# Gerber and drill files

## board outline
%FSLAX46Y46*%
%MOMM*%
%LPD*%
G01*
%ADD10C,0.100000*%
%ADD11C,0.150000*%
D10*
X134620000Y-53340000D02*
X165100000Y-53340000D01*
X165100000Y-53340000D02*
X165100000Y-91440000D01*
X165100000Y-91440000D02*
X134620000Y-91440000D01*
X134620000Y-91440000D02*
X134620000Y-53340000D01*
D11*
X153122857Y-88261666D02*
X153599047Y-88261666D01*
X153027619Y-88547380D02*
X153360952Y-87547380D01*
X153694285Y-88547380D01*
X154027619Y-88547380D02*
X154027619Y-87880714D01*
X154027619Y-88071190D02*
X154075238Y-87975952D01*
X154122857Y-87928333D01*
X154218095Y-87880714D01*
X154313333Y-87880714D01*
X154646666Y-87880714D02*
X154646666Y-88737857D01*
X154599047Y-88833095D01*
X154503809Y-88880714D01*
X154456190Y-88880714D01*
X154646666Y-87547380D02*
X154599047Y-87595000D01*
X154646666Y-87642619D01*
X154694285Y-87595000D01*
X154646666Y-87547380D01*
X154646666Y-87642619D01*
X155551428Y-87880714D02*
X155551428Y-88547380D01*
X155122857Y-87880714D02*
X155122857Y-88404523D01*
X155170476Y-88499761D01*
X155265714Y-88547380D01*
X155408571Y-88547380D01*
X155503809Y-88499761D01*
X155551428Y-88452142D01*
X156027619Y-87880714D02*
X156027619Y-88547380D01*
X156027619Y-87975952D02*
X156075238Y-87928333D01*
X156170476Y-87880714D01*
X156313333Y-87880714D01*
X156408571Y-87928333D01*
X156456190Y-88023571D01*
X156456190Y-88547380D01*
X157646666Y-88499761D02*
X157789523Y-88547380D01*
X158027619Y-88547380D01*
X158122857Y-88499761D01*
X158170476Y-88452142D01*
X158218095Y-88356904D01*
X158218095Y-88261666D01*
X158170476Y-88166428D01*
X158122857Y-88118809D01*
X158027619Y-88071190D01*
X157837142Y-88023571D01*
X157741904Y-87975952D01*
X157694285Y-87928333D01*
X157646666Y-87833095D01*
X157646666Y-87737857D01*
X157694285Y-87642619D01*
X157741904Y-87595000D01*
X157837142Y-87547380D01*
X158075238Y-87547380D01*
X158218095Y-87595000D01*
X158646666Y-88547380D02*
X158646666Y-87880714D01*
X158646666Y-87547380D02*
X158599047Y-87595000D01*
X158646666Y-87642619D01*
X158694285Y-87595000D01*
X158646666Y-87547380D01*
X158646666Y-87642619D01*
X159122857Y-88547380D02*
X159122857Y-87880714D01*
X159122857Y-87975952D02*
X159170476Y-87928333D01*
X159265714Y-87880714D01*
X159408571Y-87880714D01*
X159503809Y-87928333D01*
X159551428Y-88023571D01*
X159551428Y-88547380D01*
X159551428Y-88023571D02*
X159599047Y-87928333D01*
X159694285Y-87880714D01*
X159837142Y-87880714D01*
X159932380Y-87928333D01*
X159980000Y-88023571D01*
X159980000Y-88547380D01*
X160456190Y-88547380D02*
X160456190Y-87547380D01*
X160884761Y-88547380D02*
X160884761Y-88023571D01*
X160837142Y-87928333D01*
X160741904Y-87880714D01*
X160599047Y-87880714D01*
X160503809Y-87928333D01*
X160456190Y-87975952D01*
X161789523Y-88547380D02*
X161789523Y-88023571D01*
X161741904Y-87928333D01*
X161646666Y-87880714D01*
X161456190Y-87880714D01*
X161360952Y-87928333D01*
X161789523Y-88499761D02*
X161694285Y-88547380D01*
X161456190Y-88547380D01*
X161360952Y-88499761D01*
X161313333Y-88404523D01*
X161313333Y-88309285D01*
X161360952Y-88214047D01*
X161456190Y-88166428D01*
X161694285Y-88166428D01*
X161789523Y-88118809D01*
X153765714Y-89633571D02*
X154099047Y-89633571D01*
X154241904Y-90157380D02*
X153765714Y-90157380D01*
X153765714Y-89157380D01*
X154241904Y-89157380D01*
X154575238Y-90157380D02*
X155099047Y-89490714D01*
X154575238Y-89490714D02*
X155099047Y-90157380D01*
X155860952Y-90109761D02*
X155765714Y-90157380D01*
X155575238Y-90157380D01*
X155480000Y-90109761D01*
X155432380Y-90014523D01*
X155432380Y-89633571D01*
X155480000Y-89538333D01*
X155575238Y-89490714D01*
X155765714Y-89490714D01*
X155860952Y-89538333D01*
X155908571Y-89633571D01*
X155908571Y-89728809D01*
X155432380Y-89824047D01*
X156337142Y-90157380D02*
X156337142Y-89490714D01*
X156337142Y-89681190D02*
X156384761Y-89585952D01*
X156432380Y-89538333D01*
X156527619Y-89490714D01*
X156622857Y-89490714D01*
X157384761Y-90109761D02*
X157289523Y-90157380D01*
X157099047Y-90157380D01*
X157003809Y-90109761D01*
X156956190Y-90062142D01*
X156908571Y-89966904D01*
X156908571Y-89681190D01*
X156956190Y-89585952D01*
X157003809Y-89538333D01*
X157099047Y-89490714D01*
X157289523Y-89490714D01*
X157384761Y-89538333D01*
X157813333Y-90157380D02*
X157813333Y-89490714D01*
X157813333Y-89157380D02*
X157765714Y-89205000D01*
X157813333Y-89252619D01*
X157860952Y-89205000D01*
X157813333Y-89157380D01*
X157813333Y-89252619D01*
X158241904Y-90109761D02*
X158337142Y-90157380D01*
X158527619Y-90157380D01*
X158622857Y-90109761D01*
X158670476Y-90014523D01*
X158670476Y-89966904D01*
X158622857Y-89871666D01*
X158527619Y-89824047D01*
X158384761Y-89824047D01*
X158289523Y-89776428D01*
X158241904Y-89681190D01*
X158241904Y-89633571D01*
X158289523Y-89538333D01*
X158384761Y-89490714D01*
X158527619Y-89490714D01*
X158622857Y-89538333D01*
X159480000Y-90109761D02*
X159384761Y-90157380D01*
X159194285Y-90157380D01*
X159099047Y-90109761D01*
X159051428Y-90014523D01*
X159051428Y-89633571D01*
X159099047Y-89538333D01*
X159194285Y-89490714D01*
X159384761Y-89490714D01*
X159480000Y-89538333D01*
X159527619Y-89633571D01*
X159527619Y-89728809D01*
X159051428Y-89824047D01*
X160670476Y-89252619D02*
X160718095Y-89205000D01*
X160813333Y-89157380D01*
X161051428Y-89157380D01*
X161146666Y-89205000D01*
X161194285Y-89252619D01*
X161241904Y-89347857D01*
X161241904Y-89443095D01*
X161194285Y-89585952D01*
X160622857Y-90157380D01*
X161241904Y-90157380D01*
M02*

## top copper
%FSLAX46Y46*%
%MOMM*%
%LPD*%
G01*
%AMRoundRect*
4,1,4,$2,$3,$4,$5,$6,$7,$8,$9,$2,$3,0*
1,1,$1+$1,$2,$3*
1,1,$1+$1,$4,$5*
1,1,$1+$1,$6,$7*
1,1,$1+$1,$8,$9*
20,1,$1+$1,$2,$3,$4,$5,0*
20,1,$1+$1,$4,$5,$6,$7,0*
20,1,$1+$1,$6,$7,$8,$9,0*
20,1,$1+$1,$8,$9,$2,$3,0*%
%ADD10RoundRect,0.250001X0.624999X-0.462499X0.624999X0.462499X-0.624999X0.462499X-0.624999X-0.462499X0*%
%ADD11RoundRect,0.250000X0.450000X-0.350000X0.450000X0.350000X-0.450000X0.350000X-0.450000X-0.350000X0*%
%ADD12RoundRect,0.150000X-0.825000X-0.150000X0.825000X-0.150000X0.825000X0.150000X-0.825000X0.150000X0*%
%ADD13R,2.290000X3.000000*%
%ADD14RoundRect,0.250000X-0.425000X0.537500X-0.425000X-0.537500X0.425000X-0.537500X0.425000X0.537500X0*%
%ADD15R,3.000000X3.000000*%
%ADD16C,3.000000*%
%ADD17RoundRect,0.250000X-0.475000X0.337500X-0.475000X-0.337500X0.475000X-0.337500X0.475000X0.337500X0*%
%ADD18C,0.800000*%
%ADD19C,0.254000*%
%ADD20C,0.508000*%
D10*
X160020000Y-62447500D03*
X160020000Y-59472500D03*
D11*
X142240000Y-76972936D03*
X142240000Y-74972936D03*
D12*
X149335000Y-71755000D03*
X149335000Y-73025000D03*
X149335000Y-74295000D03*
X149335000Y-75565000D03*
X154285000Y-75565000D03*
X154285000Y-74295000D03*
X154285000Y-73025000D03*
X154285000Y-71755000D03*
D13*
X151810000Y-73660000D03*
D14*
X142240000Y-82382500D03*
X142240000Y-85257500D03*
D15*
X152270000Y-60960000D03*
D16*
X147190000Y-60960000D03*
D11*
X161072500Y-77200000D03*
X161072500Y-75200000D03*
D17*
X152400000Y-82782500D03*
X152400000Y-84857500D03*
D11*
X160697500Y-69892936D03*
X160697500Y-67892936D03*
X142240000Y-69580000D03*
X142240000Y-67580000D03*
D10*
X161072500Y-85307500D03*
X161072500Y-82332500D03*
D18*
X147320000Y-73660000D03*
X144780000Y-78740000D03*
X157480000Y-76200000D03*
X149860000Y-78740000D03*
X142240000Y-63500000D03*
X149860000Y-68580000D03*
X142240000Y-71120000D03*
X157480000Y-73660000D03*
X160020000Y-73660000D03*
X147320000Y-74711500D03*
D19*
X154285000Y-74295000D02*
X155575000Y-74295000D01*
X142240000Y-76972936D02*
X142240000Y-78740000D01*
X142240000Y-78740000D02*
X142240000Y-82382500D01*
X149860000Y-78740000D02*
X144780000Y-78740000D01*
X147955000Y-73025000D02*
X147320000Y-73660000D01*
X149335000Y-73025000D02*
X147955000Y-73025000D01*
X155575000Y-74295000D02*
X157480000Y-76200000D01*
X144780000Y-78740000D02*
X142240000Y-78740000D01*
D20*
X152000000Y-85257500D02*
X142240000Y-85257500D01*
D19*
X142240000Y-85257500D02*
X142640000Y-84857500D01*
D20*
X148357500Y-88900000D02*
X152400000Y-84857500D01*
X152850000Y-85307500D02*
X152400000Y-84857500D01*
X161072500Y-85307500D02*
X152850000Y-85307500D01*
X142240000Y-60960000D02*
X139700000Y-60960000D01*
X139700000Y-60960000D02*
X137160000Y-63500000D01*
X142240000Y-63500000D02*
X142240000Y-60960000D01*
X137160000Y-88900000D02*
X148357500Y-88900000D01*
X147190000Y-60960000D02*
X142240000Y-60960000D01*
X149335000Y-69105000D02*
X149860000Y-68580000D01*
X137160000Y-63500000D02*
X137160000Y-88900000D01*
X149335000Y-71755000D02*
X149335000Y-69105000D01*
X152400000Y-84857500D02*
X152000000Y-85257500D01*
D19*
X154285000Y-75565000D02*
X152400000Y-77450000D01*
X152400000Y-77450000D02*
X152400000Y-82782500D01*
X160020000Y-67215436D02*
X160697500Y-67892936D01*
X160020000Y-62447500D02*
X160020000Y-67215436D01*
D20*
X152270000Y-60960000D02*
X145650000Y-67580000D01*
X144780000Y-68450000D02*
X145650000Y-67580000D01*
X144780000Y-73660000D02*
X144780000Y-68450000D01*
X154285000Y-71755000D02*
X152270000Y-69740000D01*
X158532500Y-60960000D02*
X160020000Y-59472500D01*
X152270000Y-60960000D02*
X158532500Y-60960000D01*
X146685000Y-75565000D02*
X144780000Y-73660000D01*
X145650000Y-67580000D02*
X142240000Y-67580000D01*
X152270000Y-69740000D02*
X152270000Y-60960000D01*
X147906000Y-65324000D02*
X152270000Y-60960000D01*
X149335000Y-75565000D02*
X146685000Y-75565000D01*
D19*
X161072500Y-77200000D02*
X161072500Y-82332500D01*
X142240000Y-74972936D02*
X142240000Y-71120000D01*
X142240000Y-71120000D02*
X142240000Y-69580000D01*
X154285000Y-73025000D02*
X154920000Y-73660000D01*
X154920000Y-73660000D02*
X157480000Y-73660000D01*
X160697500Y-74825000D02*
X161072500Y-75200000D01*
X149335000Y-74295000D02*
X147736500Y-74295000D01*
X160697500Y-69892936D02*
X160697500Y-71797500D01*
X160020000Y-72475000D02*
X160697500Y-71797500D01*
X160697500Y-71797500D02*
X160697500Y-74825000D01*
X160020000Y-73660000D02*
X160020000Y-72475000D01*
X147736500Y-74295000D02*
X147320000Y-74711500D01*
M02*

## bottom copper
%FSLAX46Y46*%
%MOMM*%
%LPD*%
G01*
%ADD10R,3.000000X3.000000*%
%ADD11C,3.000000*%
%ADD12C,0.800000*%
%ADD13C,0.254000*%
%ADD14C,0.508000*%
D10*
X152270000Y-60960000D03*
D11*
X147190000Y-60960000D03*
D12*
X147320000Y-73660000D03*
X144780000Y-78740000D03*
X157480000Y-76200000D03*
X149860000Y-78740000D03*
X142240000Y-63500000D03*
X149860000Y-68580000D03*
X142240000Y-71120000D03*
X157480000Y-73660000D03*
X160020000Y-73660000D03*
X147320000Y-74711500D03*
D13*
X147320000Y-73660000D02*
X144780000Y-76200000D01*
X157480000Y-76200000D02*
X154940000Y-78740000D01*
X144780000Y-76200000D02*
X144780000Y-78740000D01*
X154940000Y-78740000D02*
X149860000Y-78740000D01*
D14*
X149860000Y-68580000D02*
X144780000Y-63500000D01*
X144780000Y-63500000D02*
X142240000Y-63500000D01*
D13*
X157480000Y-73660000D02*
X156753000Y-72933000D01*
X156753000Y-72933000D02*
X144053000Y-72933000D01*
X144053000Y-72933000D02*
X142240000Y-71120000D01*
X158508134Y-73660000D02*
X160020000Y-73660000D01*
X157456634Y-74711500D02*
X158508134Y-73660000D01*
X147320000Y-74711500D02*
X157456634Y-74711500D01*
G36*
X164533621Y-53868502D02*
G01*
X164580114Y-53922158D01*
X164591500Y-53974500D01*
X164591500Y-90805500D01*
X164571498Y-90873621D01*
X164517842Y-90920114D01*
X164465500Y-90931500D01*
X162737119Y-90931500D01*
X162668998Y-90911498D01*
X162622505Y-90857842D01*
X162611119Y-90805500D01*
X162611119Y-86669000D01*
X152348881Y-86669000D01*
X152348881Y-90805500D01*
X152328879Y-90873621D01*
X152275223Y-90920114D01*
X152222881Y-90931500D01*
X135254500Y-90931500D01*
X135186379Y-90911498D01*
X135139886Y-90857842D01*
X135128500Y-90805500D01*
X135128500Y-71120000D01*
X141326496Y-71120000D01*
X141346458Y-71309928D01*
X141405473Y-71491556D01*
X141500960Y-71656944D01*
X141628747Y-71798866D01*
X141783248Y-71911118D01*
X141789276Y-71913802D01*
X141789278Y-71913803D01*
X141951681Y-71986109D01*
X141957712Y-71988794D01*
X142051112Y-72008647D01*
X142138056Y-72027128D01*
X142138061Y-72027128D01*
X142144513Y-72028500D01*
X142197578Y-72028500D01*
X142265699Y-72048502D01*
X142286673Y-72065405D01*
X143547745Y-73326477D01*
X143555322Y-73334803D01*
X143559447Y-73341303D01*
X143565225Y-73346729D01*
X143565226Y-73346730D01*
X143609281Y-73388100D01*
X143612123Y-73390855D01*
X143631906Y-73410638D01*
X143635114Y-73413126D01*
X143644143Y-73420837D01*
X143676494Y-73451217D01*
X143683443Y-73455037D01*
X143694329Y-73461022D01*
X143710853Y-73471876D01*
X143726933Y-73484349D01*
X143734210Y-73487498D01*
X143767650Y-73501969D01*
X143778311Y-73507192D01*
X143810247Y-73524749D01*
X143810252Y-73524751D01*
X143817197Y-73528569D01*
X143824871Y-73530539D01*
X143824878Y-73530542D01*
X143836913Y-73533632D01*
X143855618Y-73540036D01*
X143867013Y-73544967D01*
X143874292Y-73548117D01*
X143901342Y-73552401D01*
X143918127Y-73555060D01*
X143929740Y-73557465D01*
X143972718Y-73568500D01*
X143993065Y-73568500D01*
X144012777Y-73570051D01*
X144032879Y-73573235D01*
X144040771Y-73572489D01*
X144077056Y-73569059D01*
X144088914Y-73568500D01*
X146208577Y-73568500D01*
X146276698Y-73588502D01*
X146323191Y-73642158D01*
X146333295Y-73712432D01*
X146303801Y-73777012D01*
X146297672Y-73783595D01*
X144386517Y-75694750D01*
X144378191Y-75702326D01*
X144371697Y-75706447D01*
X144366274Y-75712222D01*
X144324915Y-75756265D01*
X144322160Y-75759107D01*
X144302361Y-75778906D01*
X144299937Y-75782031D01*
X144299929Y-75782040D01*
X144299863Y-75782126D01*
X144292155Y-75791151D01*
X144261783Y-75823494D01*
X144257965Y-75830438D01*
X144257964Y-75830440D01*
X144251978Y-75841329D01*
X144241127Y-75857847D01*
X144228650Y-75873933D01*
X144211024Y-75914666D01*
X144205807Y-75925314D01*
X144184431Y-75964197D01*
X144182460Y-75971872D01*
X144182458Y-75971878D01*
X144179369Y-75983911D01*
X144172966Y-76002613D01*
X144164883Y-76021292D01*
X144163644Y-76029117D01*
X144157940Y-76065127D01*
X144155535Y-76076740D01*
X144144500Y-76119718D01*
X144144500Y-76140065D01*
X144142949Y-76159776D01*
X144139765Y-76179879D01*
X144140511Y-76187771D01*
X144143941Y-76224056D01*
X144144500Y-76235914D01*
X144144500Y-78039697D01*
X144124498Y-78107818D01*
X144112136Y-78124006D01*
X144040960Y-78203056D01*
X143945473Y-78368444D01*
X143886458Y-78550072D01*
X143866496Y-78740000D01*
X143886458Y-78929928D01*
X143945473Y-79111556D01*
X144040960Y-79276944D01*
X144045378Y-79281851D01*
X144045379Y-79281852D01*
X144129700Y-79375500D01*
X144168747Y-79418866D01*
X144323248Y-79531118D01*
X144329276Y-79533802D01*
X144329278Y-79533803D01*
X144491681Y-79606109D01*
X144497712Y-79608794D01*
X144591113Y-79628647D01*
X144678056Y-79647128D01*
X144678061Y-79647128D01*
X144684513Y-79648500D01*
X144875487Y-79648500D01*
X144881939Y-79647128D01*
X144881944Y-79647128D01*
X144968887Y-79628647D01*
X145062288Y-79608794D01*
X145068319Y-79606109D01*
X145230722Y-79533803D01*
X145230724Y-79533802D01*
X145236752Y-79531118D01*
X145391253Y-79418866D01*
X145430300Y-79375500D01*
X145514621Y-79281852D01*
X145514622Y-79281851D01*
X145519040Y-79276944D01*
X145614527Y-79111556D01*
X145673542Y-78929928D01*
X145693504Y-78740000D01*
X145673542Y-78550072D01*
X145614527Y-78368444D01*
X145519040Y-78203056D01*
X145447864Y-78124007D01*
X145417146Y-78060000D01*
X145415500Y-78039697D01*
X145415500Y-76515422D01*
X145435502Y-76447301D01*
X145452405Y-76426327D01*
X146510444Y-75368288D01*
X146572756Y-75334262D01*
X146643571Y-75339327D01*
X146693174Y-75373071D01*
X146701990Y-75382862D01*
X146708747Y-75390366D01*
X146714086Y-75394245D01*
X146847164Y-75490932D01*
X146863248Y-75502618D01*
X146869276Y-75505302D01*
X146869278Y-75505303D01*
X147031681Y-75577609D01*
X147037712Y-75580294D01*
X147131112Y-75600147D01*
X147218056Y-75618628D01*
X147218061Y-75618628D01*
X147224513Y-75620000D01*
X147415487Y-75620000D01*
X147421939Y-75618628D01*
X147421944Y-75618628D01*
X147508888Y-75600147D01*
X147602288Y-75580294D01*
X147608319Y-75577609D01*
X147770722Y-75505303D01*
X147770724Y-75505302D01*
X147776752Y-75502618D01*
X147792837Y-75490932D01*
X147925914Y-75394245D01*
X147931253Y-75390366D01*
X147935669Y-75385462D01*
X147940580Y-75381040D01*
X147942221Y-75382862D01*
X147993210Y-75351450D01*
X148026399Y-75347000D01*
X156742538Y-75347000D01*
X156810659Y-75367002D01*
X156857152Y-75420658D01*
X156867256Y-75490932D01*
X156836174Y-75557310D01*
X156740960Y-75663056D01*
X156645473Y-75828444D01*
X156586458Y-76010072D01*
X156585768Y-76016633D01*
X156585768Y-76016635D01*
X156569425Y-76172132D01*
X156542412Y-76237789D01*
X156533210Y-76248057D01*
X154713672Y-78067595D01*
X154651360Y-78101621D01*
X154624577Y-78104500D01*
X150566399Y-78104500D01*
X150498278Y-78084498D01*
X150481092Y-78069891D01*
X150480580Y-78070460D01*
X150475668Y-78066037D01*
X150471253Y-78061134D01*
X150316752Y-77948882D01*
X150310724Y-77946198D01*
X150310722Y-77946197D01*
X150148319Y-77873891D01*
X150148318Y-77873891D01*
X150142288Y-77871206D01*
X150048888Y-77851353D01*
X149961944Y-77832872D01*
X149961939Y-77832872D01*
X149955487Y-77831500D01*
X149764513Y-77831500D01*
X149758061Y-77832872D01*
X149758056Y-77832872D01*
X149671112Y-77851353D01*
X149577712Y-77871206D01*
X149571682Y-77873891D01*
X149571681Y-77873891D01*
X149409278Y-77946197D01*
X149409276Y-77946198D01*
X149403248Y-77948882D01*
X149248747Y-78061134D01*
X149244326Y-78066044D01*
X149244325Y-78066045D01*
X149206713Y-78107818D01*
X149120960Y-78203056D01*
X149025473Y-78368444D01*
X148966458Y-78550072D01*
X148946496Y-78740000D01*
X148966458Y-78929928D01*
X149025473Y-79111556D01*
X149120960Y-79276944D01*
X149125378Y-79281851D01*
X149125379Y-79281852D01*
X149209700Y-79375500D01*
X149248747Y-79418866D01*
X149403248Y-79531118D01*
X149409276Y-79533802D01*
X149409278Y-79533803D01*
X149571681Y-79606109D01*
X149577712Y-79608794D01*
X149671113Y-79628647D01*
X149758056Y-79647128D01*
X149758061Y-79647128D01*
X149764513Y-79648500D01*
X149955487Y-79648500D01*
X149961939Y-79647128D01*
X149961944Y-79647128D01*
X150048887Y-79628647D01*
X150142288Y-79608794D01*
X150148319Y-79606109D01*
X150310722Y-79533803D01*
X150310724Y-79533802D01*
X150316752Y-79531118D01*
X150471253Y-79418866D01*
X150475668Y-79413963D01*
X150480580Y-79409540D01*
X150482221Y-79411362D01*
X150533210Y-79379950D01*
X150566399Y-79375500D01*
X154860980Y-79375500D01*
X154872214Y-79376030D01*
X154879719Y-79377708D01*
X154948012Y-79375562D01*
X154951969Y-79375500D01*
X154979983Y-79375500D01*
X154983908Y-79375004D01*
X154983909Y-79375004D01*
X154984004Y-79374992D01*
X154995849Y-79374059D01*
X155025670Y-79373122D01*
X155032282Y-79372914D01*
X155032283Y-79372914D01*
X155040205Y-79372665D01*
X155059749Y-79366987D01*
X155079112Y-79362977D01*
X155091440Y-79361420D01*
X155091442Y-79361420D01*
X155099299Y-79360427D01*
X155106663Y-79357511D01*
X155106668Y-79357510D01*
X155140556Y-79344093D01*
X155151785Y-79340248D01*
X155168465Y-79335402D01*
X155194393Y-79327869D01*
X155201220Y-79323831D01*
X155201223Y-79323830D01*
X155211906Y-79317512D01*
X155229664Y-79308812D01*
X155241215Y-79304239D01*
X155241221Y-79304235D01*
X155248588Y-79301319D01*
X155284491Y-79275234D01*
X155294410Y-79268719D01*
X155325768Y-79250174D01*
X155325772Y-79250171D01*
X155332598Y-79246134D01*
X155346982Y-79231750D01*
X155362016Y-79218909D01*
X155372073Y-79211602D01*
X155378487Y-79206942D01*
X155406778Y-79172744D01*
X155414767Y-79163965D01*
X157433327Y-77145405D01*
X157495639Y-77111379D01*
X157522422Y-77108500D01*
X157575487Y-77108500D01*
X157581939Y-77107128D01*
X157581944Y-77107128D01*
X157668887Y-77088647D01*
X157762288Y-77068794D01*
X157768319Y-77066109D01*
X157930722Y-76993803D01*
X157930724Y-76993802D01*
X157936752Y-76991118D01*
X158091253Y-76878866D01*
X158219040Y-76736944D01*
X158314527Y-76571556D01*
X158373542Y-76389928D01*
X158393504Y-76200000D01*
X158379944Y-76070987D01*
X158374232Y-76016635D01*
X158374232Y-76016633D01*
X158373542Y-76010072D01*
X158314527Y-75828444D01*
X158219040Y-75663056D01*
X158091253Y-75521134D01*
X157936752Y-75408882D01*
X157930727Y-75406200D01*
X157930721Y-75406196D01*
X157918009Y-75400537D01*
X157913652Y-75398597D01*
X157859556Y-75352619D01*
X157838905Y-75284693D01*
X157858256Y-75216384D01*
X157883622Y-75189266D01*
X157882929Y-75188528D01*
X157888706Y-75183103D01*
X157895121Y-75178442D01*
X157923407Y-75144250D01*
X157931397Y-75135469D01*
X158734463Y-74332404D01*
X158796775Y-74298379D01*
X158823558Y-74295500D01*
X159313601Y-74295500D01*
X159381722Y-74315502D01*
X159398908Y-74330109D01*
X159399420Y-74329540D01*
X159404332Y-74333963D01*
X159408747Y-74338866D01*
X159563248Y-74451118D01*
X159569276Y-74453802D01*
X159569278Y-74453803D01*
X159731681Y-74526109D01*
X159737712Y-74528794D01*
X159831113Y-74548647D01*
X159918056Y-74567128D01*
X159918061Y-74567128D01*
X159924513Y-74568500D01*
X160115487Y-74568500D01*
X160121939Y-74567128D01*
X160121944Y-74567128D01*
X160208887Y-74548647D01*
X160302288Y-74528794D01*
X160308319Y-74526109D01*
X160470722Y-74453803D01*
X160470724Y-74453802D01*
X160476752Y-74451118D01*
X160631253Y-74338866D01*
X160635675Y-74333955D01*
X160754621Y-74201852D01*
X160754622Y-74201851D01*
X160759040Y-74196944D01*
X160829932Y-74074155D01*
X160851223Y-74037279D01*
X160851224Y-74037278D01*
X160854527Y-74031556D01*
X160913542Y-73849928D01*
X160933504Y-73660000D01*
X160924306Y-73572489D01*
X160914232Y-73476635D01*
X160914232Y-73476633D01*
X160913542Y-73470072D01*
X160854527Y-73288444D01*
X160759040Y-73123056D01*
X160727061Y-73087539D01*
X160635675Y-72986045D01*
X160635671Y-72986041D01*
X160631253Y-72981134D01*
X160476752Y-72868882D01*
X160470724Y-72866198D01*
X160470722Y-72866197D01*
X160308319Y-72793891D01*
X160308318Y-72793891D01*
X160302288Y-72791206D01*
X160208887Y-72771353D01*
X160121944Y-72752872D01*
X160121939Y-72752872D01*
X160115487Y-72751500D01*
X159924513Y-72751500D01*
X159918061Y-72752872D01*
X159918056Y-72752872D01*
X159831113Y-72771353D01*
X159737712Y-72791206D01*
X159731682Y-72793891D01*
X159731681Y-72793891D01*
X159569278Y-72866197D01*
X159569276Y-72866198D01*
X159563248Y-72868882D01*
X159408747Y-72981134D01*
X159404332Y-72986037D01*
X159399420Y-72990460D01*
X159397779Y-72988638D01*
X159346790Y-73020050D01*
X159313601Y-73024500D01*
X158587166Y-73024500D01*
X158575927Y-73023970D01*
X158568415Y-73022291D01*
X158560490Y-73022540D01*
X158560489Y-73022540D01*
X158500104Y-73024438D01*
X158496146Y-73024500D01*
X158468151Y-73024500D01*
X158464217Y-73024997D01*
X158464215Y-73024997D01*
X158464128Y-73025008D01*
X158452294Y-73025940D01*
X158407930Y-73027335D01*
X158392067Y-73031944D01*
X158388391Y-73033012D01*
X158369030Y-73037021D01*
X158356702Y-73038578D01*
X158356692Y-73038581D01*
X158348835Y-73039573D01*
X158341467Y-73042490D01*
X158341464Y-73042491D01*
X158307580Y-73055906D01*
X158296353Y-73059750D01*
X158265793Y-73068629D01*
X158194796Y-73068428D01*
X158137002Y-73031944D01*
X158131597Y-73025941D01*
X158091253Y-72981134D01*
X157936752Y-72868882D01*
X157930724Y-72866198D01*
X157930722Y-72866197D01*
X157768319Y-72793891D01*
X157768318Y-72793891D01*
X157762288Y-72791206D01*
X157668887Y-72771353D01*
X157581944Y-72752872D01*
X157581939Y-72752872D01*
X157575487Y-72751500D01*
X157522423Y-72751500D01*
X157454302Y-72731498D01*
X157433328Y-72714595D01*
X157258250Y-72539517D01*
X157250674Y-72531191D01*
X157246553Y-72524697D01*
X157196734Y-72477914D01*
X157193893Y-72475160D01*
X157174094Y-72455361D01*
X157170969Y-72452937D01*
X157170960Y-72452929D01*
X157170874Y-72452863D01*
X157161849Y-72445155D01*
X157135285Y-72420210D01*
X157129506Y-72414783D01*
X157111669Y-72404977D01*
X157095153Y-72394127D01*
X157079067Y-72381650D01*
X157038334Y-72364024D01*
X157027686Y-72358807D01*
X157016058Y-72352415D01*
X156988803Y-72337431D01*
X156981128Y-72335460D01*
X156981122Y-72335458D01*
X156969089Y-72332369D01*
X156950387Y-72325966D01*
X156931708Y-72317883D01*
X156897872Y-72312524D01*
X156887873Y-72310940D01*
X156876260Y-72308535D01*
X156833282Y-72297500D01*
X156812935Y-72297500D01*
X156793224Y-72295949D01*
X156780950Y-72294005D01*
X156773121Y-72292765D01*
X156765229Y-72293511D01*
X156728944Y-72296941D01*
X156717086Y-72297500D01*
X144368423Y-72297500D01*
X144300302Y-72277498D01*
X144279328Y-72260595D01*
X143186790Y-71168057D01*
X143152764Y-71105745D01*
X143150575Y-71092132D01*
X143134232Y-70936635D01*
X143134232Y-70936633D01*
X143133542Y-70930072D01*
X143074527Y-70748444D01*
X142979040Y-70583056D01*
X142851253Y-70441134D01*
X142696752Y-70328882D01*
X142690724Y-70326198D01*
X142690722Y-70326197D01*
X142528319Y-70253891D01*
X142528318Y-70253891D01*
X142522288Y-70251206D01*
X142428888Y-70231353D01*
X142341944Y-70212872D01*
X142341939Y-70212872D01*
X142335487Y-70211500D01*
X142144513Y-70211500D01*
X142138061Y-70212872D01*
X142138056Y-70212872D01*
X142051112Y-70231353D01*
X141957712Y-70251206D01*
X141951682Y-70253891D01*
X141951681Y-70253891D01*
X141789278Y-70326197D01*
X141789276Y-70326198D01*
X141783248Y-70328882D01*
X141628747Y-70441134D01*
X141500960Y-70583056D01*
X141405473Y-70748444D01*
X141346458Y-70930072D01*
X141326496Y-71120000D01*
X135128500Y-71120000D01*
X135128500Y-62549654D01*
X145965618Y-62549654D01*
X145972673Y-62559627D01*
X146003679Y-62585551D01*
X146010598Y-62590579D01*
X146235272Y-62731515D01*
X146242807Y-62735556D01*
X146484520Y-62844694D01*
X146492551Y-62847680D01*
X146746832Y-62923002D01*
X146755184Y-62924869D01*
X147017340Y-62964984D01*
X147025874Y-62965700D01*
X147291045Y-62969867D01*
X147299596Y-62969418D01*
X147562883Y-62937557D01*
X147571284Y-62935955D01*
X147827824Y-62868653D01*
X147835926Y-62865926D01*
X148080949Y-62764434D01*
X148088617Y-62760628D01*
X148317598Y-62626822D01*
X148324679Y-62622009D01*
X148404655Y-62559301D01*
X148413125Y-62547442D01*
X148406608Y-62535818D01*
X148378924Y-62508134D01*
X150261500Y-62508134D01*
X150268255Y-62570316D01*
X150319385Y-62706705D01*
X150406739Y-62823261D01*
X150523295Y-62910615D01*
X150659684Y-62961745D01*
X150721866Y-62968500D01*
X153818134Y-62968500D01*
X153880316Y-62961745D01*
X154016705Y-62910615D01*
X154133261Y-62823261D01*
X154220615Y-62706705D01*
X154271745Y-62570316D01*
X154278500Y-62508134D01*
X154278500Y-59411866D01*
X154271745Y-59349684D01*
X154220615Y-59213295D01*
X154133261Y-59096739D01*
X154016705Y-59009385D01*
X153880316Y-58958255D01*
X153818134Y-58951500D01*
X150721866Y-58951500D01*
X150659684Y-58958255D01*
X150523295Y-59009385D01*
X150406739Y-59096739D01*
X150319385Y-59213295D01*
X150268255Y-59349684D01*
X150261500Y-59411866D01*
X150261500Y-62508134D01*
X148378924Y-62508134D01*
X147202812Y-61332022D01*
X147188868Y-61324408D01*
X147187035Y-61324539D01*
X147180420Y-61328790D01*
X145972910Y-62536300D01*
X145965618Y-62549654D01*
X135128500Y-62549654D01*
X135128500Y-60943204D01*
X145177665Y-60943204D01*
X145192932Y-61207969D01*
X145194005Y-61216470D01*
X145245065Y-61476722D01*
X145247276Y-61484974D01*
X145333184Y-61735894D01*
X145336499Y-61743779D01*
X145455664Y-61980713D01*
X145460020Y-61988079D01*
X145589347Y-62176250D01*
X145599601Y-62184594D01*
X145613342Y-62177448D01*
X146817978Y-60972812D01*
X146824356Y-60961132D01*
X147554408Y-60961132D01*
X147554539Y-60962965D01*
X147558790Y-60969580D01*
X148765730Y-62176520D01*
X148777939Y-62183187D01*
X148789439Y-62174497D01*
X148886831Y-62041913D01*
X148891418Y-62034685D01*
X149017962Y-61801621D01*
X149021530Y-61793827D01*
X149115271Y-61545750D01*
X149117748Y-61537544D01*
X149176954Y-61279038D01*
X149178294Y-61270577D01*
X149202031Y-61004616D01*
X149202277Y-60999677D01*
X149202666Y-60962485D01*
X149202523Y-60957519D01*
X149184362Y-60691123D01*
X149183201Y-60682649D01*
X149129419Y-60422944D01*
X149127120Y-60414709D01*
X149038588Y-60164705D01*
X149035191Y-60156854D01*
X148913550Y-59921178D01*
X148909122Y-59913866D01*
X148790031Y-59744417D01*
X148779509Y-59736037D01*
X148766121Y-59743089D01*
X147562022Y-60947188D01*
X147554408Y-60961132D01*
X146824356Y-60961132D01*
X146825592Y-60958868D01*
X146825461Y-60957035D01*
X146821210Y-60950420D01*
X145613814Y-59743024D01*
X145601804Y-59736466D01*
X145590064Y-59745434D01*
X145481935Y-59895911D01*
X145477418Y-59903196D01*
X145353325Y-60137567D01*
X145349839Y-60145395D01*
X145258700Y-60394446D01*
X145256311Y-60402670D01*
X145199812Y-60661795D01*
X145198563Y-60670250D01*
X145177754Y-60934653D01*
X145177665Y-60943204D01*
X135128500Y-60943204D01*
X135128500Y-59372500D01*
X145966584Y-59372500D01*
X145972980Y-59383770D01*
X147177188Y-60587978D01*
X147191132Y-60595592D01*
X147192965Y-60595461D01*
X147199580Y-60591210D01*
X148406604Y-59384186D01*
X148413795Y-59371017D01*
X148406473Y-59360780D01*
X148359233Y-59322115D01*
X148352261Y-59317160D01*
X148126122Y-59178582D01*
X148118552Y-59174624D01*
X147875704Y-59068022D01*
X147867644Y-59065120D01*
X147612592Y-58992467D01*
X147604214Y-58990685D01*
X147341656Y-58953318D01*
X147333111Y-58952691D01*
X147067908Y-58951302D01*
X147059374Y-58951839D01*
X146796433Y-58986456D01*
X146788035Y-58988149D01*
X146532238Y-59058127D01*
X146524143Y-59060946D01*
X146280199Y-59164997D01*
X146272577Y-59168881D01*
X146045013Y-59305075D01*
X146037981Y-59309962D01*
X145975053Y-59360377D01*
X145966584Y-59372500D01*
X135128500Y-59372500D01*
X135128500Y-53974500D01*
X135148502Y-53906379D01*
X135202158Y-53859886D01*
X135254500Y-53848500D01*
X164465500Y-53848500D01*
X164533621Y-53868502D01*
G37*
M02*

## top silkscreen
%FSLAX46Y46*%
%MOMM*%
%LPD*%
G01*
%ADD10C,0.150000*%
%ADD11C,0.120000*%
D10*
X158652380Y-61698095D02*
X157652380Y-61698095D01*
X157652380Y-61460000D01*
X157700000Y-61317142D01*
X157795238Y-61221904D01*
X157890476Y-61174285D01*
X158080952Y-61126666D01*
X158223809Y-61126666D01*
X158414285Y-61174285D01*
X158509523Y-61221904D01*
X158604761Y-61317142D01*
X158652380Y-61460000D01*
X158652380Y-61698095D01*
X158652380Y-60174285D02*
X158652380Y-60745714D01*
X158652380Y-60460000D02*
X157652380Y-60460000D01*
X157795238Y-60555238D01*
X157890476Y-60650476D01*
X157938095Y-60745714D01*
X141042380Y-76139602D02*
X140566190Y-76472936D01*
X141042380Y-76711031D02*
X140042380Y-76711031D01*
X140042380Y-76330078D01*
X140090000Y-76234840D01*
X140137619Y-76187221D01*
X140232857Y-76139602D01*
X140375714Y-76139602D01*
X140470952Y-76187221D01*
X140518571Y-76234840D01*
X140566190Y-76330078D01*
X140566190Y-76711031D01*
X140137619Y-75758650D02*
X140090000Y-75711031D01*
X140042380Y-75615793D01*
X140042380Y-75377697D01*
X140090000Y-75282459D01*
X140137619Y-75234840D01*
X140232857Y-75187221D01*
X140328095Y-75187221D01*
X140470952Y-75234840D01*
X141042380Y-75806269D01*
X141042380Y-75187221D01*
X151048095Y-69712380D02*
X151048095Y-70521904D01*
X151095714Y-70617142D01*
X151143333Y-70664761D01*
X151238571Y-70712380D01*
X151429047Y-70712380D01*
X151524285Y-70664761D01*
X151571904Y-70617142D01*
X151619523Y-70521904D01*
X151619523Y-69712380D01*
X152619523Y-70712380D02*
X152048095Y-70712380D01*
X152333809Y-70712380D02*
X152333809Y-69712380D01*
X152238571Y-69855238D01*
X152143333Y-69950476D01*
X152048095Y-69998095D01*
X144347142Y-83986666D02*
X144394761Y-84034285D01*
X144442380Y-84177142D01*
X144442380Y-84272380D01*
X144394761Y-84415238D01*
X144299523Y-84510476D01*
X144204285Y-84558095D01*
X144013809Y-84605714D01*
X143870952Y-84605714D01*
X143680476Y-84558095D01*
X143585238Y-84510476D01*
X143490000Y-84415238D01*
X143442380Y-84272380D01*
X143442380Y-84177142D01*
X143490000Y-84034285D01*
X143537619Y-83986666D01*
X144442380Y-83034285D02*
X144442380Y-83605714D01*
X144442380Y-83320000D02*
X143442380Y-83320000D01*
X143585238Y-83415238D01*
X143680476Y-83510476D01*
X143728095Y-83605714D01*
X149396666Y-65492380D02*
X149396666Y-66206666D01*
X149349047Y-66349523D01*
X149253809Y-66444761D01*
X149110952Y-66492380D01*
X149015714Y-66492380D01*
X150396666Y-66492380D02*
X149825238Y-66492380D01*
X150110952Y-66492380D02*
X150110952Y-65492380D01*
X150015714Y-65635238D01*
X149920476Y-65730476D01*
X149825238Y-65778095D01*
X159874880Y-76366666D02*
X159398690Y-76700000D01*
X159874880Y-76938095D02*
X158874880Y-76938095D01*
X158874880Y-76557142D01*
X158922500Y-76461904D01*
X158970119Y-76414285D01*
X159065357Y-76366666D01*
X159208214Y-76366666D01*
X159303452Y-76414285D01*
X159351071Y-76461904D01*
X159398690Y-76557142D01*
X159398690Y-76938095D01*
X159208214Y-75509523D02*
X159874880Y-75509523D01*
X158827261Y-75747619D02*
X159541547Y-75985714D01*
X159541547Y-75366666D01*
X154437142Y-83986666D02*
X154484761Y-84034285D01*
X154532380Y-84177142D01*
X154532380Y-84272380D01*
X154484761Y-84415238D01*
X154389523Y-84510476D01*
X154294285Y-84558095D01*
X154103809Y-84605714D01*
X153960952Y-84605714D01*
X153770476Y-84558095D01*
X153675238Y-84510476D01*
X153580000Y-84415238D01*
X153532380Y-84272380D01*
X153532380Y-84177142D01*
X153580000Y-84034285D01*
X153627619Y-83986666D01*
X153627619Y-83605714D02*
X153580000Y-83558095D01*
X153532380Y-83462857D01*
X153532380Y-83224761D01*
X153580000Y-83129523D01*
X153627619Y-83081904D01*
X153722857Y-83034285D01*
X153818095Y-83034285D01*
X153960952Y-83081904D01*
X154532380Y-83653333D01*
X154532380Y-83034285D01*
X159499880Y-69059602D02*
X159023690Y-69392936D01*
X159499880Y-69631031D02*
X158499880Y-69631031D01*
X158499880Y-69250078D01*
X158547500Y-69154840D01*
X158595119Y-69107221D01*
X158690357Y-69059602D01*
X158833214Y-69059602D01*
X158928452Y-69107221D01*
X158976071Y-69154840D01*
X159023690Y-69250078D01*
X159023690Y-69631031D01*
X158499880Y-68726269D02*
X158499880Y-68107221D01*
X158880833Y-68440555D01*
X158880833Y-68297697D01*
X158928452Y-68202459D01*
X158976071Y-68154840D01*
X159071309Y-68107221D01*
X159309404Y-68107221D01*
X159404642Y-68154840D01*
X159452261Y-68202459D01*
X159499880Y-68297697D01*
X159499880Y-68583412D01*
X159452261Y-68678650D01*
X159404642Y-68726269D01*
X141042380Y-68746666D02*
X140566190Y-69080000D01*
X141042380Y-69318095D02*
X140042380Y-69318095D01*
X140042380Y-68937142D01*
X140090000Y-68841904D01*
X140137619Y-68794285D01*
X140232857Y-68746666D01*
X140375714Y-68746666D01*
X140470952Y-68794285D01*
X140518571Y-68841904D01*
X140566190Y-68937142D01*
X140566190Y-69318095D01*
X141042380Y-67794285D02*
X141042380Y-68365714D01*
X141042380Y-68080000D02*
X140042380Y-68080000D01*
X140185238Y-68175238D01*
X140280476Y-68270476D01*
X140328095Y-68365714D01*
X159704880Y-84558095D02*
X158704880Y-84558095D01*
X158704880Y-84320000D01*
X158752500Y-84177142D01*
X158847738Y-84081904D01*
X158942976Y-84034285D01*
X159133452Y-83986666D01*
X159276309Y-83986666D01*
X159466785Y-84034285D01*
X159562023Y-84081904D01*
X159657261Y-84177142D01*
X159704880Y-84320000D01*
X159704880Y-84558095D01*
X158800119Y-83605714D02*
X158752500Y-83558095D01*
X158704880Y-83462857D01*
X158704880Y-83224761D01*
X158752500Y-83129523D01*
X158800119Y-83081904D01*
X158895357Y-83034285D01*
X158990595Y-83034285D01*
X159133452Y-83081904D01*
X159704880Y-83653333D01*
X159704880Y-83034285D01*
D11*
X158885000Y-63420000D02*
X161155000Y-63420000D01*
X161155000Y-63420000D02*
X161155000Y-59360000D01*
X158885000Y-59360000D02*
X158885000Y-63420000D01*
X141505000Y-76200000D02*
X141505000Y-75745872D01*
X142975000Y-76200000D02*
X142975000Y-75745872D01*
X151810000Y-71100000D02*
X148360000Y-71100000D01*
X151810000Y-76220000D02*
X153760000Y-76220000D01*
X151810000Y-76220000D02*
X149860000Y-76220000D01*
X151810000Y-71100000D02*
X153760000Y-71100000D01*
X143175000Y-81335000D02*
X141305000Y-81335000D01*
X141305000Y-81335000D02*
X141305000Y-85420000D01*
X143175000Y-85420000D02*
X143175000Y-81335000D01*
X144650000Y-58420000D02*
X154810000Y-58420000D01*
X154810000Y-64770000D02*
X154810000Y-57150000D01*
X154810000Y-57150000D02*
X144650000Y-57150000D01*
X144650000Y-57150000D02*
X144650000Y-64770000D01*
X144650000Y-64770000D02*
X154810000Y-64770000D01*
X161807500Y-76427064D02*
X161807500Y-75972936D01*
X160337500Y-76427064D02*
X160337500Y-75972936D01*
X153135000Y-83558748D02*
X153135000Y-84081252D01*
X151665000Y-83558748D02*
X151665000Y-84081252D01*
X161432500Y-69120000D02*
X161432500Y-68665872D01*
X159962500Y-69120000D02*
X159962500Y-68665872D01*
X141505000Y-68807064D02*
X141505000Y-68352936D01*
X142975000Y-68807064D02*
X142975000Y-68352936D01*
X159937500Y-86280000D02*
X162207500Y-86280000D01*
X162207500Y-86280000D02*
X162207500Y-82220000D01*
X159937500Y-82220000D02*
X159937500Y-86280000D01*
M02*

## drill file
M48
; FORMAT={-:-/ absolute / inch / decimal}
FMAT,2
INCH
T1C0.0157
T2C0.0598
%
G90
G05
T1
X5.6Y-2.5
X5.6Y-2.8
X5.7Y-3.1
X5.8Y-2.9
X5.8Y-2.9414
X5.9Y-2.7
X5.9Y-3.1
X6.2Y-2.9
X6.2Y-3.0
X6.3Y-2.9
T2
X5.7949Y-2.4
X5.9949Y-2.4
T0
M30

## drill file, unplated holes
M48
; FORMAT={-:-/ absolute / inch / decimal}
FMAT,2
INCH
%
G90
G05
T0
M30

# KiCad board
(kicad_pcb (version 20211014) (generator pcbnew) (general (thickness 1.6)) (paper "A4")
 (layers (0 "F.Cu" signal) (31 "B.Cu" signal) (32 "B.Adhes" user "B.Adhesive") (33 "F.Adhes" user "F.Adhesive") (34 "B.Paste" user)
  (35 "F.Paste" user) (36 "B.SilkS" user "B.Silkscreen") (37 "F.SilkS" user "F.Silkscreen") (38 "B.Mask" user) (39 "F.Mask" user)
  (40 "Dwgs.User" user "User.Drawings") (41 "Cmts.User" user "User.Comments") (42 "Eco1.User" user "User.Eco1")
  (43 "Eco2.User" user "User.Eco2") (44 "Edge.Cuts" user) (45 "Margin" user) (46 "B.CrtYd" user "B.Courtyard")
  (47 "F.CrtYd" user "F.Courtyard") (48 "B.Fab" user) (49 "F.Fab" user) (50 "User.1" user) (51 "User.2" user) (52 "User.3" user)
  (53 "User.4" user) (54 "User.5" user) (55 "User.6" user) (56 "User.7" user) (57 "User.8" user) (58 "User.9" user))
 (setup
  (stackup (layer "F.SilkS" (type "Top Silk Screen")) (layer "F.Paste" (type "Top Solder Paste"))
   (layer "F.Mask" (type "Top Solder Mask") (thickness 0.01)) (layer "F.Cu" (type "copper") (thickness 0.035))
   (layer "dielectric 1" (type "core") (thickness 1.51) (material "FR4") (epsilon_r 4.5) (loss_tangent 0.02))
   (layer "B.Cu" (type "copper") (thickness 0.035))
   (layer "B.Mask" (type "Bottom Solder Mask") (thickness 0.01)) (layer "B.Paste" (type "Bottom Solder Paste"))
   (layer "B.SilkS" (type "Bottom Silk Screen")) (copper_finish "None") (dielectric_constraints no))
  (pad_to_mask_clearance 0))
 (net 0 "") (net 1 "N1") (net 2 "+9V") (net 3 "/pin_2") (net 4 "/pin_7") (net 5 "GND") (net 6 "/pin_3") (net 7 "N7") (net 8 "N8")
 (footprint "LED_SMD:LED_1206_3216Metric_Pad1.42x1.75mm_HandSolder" (layer "F.Cu") (at 160.02 60.96 90)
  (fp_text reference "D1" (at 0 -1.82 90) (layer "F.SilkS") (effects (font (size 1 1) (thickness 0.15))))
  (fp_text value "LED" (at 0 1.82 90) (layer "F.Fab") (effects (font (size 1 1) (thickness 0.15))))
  (fp_line (start -2.46 -1.135) (end -2.46 1.135) (layer "F.SilkS") (width 0.12))
  (fp_line (start -2.46 1.135) (end 1.6 1.135) (layer "F.SilkS") (width 0.12))
  (fp_line (start 1.6 -1.135) (end -2.46 -1.135) (layer "F.SilkS") (width 0.12))
  (pad "1" smd roundrect (at -1.4875 0 90) (size 1.425 1.75) (layers "F.Cu" "F.Paste" "F.Mask") (roundrect_rratio 0.1754392982) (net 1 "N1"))
  (pad "2" smd roundrect (at 1.4875 0 90) (size 1.425 1.75) (layers "F.Cu" "F.Paste" "F.Mask") (roundrect_rratio 0.1754392982) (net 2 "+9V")))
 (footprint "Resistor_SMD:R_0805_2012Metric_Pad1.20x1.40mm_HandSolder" (layer "F.Cu") (at 142.24 75.972936 90)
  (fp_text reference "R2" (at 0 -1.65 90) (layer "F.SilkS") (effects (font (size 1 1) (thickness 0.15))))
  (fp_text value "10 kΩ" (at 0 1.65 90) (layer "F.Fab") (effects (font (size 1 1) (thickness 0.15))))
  (fp_line (start -0.227064 -0.735) (end 0.227064 -0.735) (layer "F.SilkS") (width 0.12))
  (fp_line (start -0.227064 0.735) (end 0.227064 0.735) (layer "F.SilkS") (width 0.12))
  (pad "1" smd roundrect (at -1 0 90) (size 1.2 1.4) (layers "F.Cu" "F.Paste" "F.Mask") (roundrect_rratio 0.2083333333) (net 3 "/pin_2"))
  (pad "2" smd roundrect (at 1 0 90) (size 1.2 1.4) (layers "F.Cu" "F.Paste" "F.Mask") (roundrect_rratio 0.2083333333) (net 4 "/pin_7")))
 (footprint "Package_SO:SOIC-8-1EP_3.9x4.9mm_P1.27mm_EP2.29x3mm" (layer "F.Cu") (at 151.81 73.66)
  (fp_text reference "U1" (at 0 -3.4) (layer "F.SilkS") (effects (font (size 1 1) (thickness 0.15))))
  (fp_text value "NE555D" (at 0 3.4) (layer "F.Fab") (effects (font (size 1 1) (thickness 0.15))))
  (fp_line (start 0 -2.56) (end -3.45 -2.56) (layer "F.SilkS") (width 0.12))
  (fp_line (start 0 2.56) (end 1.95 2.56) (layer "F.SilkS") (width 0.12))
  (fp_line (start 0 2.56) (end -1.95 2.56) (layer "F.SilkS") (width 0.12))
  (fp_line (start 0 -2.56) (end 1.95 -2.56) (layer "F.SilkS") (width 0.12))
  (pad "" smd roundrect (at -0.57 0.75) (size 0.92 1.21) (layers "F.Paste") (roundrect_rratio 0.25))
  (pad "" smd roundrect (at -0.57 -0.75) (size 0.92 1.21) (layers "F.Paste") (roundrect_rratio 0.25))
  (pad "" smd roundrect (at 0.57 -0.75) (size 0.92 1.21) (layers "F.Paste") (roundrect_rratio 0.25))
  (pad "" smd roundrect (at 0.57 0.75) (size 0.92 1.21) (layers "F.Paste") (roundrect_rratio 0.25))
  (pad "1" smd roundrect (at -2.475 -1.905) (size 1.95 0.6) (layers "F.Cu" "F.Paste" "F.Mask") (roundrect_rratio 0.25) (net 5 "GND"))
  (pad "2" smd roundrect (at -2.475 -0.635) (size 1.95 0.6) (layers "F.Cu" "F.Paste" "F.Mask") (roundrect_rratio 0.25) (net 3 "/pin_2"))
  (pad "3" smd roundrect (at -2.475 0.635) (size 1.95 0.6) (layers "F.Cu" "F.Paste" "F.Mask") (roundrect_rratio 0.25) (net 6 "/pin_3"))
  (pad "4" smd roundrect (at -2.475 1.905) (size 1.95 0.6) (layers "F.Cu" "F.Paste" "F.Mask") (roundrect_rratio 0.25) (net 2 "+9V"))
  (pad "5" smd roundrect (at 2.475 1.905) (size 1.95 0.6) (layers "F.Cu" "F.Paste" "F.Mask") (roundrect_rratio 0.25) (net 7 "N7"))
  (pad "6" smd roundrect (at 2.475 0.635) (size 1.95 0.6) (layers "F.Cu" "F.Paste" "F.Mask") (roundrect_rratio 0.25) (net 3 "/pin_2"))
  (pad "7" smd roundrect (at 2.475 -0.635) (size 1.95 0.6) (layers "F.Cu" "F.Paste" "F.Mask") (roundrect_rratio 0.25) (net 4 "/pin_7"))
  (pad "8" smd roundrect (at 2.475 -1.905) (size 1.95 0.6) (layers "F.Cu" "F.Paste" "F.Mask") (roundrect_rratio 0.25) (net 2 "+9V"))
  (pad "9" smd rect (at 0 0) (size 2.29 3) (layers "F.Cu" "F.Mask")))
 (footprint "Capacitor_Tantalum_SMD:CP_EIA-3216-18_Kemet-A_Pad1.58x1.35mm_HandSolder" (layer "F.Cu") (at 142.24 83.82 -90)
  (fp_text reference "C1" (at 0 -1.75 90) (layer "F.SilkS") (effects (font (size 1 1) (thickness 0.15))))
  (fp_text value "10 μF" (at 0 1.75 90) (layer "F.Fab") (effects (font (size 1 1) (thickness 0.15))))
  (fp_line (start -2.485 -0.935) (end -2.485 0.935) (layer "F.SilkS") (width 0.12))
  (fp_line (start -2.485 0.935) (end 1.6 0.935) (layer "F.SilkS") (width 0.12))
  (fp_line (start 1.6 -0.935) (end -2.485 -0.935) (layer "F.SilkS") (width 0.12))
  (pad "1" smd roundrect (at -1.4375 0 270) (size 1.575 1.35) (layers "F.Cu" "F.Paste" "F.Mask") (roundrect_rratio 0.1851851852)
   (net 3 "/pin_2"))
  (pad "2" smd roundrect (at 1.4375 0 270) (size 1.575 1.35) (layers "F.Cu" "F.Paste" "F.Mask") (roundrect_rratio 0.1851851852)
   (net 5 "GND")))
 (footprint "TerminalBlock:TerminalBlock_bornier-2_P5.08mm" (layer "F.Cu") (at 152.27 60.96 180)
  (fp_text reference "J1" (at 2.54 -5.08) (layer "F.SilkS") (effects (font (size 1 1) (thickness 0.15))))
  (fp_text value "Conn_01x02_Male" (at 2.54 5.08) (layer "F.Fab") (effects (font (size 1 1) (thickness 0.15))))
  (fp_line (start 7.62 2.54) (end -2.54 2.54) (layer "F.SilkS") (width 0.12))
  (fp_line (start -2.54 -3.81) (end -2.54 3.81) (layer "F.SilkS") (width 0.12))
  (fp_line (start -2.54 3.81) (end 7.62 3.81) (layer "F.SilkS") (width 0.12))
  (fp_line (start 7.62 3.81) (end 7.62 -3.81) (layer "F.SilkS") (width 0.12))
  (fp_line (start 7.62 -3.81) (end -2.54 -3.81) (layer "F.SilkS") (width 0.12))
  (pad "1" thru_hole rect (at 0 0 180) (size 3 3) (drill 1.52) (layers *.Cu *.Mask) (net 2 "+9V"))
  (pad "2" thru_hole circle (at 5.08 0 180) (size 3 3) (drill 1.52) (layers *.Cu *.Mask) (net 5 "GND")))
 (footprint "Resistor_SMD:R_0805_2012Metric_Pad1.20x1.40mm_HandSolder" (layer "F.Cu") (at 161.0725 76.2 90)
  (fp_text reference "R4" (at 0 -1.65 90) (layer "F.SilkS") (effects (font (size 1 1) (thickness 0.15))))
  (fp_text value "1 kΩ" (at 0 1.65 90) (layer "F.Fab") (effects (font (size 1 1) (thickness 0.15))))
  (fp_line (start -0.227064 0.735) (end 0.227064 0.735) (layer "F.SilkS") (width 0.12))
  (fp_line (start -0.227064 -0.735) (end 0.227064 -0.735) (layer "F.SilkS") (width 0.12))
  (pad "1" smd roundrect (at -1 0 90) (size 1.2 1.4) (layers "F.Cu" "F.Paste" "F.Mask") (roundrect_rratio 0.2083333333) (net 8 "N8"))
  (pad "2" smd roundrect (at 1 0 90) (size 1.2 1.4) (layers "F.Cu" "F.Paste" "F.Mask") (roundrect_rratio 0.2083333333) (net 6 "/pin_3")))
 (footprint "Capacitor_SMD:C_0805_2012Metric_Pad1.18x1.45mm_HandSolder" (layer "F.Cu") (at 152.4 83.82 -90)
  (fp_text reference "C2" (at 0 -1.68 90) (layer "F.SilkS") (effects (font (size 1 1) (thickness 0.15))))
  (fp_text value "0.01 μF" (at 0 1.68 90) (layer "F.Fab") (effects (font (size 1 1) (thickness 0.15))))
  (fp_line (start -0.261252 -0.735) (end 0.261252 -0.735) (layer "F.SilkS") (width 0.12))
  (fp_line (start -0.261252 0.735) (end 0.261252 0.735) (layer "F.SilkS") (width 0.12))
  (pad "1" smd roundrect (at -1.0375 0 270) (size 1.175 1.45) (layers "F.Cu" "F.Paste" "F.Mask") (roundrect_rratio 0.2127659574)
   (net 7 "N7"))
  (pad "2" smd roundrect (at 1.0375 0 270) (size 1.175 1.45) (layers "F.Cu" "F.Paste" "F.Mask") (roundrect_rratio 0.2127659574)
   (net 5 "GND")))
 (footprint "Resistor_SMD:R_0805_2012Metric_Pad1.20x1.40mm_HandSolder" (layer "F.Cu") (at 160.6975 68.892936 90)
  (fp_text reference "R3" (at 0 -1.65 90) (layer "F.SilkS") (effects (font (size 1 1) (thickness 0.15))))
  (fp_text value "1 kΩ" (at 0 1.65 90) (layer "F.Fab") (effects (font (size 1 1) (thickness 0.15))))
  (fp_line (start -0.227064 0.735) (end 0.227064 0.735) (layer "F.SilkS") (width 0.12))
  (fp_line (start -0.227064 -0.735) (end 0.227064 -0.735) (layer "F.SilkS") (width 0.12))
  (pad "1" smd roundrect (at -1 0 90) (size 1.2 1.4) (layers "F.Cu" "F.Paste" "F.Mask") (roundrect_rratio 0.2083333333) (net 6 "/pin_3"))
  (pad "2" smd roundrect (at 1 0 90) (size 1.2 1.4) (layers "F.Cu" "F.Paste" "F.Mask") (roundrect_rratio 0.2083333333) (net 1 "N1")))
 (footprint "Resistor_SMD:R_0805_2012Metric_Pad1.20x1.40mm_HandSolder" (layer "F.Cu") (at 142.24 68.58 90)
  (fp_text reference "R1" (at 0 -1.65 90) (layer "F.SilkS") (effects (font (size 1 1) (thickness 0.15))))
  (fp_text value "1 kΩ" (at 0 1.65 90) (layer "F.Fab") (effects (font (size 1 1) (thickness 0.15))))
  (fp_line (start -0.227064 -0.735) (end 0.227064 -0.735) (layer "F.SilkS") (width 0.12))
  (fp_line (start -0.227064 0.735) (end 0.227064 0.735) (layer "F.SilkS") (width 0.12))
  (pad "1" smd roundrect (at -1 0 90) (size 1.2 1.4) (layers "F.Cu" "F.Paste" "F.Mask") (roundrect_rratio 0.2083333333) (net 4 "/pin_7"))
  (pad "2" smd roundrect (at 1 0 90) (size 1.2 1.4) (layers "F.Cu" "F.Paste" "F.Mask") (roundrect_rratio 0.2083333333) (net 2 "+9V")))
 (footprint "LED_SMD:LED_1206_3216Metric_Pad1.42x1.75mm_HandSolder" (layer "F.Cu") (at 161.0725 83.82 90)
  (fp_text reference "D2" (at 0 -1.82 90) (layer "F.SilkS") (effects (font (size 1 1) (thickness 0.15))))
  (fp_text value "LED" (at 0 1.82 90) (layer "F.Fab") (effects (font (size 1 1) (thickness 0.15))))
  (fp_line (start -2.46 -1.135) (end -2.46 1.135) (layer "F.SilkS") (width 0.12))
  (fp_line (start -2.46 1.135) (end 1.6 1.135) (layer "F.SilkS") (width 0.12))
  (fp_line (start 1.6 -1.135) (end -2.46 -1.135) (layer "F.SilkS") (width 0.12))
  (pad "1" smd roundrect (at -1.4875 0 90) (size 1.425 1.75) (layers "F.Cu" "F.Paste" "F.Mask") (roundrect_rratio 0.1754392982)
   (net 5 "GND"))
  (pad "2" smd roundrect (at 1.4875 0 90) (size 1.425 1.75) (layers "F.Cu" "F.Paste" "F.Mask") (roundrect_rratio 0.1754392982) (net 8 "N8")))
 (gr_rect (start 134.62 53.34) (end 165.1 91.44) (layer "Edge.Cuts") (width 0.1) (fill none))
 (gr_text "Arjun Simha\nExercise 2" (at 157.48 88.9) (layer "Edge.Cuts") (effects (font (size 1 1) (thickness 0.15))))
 (segment (start 154.285 74.295) (end 155.575 74.295) (width 0.254) (layer "F.Cu") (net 3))
 (segment (start 142.24 76.972936) (end 142.24 78.74) (width 0.254) (layer "F.Cu") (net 3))
 (segment (start 142.24 78.74) (end 142.24 82.3825) (width 0.254) (layer "F.Cu") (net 3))
 (segment (start 149.86 78.74) (end 144.78 78.74) (width 0.254) (layer "F.Cu") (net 3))
 (segment (start 147.955 73.025) (end 147.32 73.66) (width 0.254) (layer "F.Cu") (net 3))
 (segment (start 149.335 73.025) (end 147.955 73.025) (width 0.254) (layer "F.Cu") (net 3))
 (segment (start 155.575 74.295) (end 157.48 76.2) (width 0.254) (layer "F.Cu") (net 3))
 (segment (start 144.78 78.74) (end 142.24 78.74) (width 0.254) (layer "F.Cu") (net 3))
 (via (at 147.32 73.66) (size 0.8) (drill 0.4) (layers "F.Cu" "B.Cu") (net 3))
 (via (at 144.78 78.74) (size 0.8) (drill 0.4) (layers "F.Cu" "B.Cu") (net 3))
 (via (at 157.48 76.2) (size 0.8) (drill 0.4) (layers "F.Cu" "B.Cu") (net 3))
 (via (at 149.86 78.74) (size 0.8) (drill 0.4) (layers "F.Cu" "B.Cu") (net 3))
 (segment (start 147.32 73.66) (end 144.78 76.2) (width 0.254) (layer "B.Cu") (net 3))
 (segment (start 157.48 76.2) (end 154.94 78.74) (width 0.254) (layer "B.Cu") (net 3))
 (segment (start 144.78 76.2) (end 144.78 78.74) (width 0.254) (layer "B.Cu") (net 3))
 (segment (start 154.94 78.74) (end 149.86 78.74) (width 0.254) (layer "B.Cu") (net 3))
 (segment (start 152 85.2575) (end 142.24 85.2575) (width 0.508) (layer "F.Cu") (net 5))
 (segment (start 142.24 85.2575) (end 142.64 84.8575) (width 0.254) (layer "F.Cu") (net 5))
 (segment (start 148.3575 88.9) (end 152.4 84.8575) (width 0.508) (layer "F.Cu") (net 5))
 (segment (start 152.85 85.3075) (end 152.4 84.8575) (width 0.508) (layer "F.Cu") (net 5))
 (segment (start 161.0725 85.3075) (end 152.85 85.3075) (width 0.508) (layer "F.Cu") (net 5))
 (segment (start 142.24 60.96) (end 139.7 60.96) (width 0.508) (layer "F.Cu") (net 5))
 (segment (start 139.7 60.96) (end 137.16 63.5) (width 0.508) (layer "F.Cu") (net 5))
 (segment (start 142.24 63.5) (end 142.24 60.96) (width 0.508) (layer "F.Cu") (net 5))
 (segment (start 137.16 88.9) (end 148.3575 88.9) (width 0.508) (layer "F.Cu") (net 5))
 (segment (start 147.19 60.96) (end 142.24 60.96) (width 0.508) (layer "F.Cu") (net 5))
 (segment (start 149.335 69.105) (end 149.86 68.58) (width 0.508) (layer "F.Cu") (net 5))
 (segment (start 137.16 63.5) (end 137.16 88.9) (width 0.508) (layer "F.Cu") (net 5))
 (segment (start 149.335 71.755) (end 149.335 69.105) (width 0.508) (layer "F.Cu") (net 5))
 (segment (start 152.4 84.8575) (end 152 85.2575) (width 0.508) (layer "F.Cu") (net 5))
 (via (at 142.24 63.5) (size 0.8) (drill 0.4) (layers "F.Cu" "B.Cu") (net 5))
 (via (at 149.86 68.58) (size 0.8) (drill 0.4) (layers "F.Cu" "B.Cu") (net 5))
 (segment (start 149.86 68.58) (end 144.78 63.5) (width 0.508) (layer "B.Cu") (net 5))
 (segment (start 144.78 63.5) (end 142.24 63.5) (width 0.508) (layer "B.Cu") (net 5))
 (segment (start 154.285 75.565) (end 152.4 77.45) (width 0.254) (layer "F.Cu") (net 7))
 (segment (start 152.4 77.45) (end 152.4 82.7825) (width 0.254) (layer "F.Cu") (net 7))
 (segment (start 160.02 67.215436) (end 160.6975 67.892936) (width 0.254) (layer "F.Cu") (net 1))
 (segment (start 160.02 62.4475) (end 160.02 67.215436) (width 0.254) (layer "F.Cu") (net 1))
 (segment (start 152.27 60.96) (end 145.65 67.58) (width 0.508) (layer "F.Cu") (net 2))
 (segment (start 144.78 68.45) (end 145.65 67.58) (width 0.508) (layer "F.Cu") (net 2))
 (segment (start 144.78 73.66) (end 144.78 68.45) (width 0.508) (layer "F.Cu") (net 2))
 (segment (start 154.285 71.755) (end 152.27 69.74) (width 0.508) (layer "F.Cu") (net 2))
 (segment (start 158.5325 60.96) (end 160.02 59.4725) (width 0.508) (layer "F.Cu") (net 2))
 (segment (start 152.27 60.96) (end 158.5325 60.96) (width 0.508) (layer "F.Cu") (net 2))
 (segment (start 146.685 75.565) (end 144.78 73.66) (width 0.508) (layer "F.Cu") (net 2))
 (segment (start 145.65 67.58) (end 142.24 67.58) (width 0.508) (layer "F.Cu") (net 2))
 (segment (start 152.27 69.74) (end 152.27 60.96) (width 0.508) (layer "F.Cu") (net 2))
 (segment (start 147.906 65.324) (end 152.27 60.96) (width 0.508) (layer "F.Cu") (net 2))
 (segment (start 149.335 75.565) (end 146.685 75.565) (width 0.508) (layer "F.Cu") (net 2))
 (segment (start 161.0725 77.2) (end 161.0725 82.3325) (width 0.254) (layer "F.Cu") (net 8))
 (segment (start 142.24 74.972936) (end 142.24 71.12) (width 0.254) (layer "F.Cu") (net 4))
 (segment (start 142.24 71.12) (end 142.24 69.58) (width 0.254) (layer "F.Cu") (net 4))
 (segment (start 154.285 73.025) (end 154.92 73.66) (width 0.254) (layer "F.Cu") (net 4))
 (segment (start 154.92 73.66) (end 157.48 73.66) (width 0.254) (layer "F.Cu") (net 4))
 (via (at 142.24 71.12) (size 0.8) (drill 0.4) (layers "F.Cu" "B.Cu") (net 4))
 (via (at 157.48 73.66) (size 0.8) (drill 0.4) (layers "F.Cu" "B.Cu") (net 4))
 (segment (start 157.48 73.66) (end 156.753 72.933) (width 0.254) (layer "B.Cu") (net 4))
 (segment (start 156.753 72.933) (end 144.053 72.933) (width 0.254) (layer "B.Cu") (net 4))
 (segment (start 144.053 72.933) (end 142.24 71.12) (width 0.254) (layer "B.Cu") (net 4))
 (segment (start 160.6975 74.825) (end 161.0725 75.2) (width 0.254) (layer "F.Cu") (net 6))
 (segment (start 149.335 74.295) (end 147.7365 74.295) (width 0.254) (layer "F.Cu") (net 6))
 (segment (start 160.6975 69.892936) (end 160.6975 71.7975) (width 0.254) (layer "F.Cu") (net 6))
 (segment (start 160.02 72.475) (end 160.6975 71.7975) (width 0.254) (layer "F.Cu") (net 6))
 (segment (start 160.6975 71.7975) (end 160.6975 74.825) (width 0.254) (layer "F.Cu") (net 6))
 (segment (start 160.02 73.66) (end 160.02 72.475) (width 0.254) (layer "F.Cu") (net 6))
 (segment (start 147.7365 74.295) (end 147.32 74.7115) (width 0.254) (layer "F.Cu") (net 6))
 (via (at 160.02 73.66) (size 0.8) (drill 0.4) (layers "F.Cu" "B.Cu") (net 6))
 (via (at 147.32 74.7115) (size 0.8) (drill 0.4) (layers "F.Cu" "B.Cu") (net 6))
 (segment (start 158.508134 73.66) (end 160.02 73.66) (width 0.254) (layer "B.Cu") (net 6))
 (segment (start 157.456634 74.7115) (end 158.508134 73.66) (width 0.254) (layer "B.Cu") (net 6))
 (segment (start 147.32 74.7115) (end 157.456634 74.7115) (width 0.254) (layer "B.Cu") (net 6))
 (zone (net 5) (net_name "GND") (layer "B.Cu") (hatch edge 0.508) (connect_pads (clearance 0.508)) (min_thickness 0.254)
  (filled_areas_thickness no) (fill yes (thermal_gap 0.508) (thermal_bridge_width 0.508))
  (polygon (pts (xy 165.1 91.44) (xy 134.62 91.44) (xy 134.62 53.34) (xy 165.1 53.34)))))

